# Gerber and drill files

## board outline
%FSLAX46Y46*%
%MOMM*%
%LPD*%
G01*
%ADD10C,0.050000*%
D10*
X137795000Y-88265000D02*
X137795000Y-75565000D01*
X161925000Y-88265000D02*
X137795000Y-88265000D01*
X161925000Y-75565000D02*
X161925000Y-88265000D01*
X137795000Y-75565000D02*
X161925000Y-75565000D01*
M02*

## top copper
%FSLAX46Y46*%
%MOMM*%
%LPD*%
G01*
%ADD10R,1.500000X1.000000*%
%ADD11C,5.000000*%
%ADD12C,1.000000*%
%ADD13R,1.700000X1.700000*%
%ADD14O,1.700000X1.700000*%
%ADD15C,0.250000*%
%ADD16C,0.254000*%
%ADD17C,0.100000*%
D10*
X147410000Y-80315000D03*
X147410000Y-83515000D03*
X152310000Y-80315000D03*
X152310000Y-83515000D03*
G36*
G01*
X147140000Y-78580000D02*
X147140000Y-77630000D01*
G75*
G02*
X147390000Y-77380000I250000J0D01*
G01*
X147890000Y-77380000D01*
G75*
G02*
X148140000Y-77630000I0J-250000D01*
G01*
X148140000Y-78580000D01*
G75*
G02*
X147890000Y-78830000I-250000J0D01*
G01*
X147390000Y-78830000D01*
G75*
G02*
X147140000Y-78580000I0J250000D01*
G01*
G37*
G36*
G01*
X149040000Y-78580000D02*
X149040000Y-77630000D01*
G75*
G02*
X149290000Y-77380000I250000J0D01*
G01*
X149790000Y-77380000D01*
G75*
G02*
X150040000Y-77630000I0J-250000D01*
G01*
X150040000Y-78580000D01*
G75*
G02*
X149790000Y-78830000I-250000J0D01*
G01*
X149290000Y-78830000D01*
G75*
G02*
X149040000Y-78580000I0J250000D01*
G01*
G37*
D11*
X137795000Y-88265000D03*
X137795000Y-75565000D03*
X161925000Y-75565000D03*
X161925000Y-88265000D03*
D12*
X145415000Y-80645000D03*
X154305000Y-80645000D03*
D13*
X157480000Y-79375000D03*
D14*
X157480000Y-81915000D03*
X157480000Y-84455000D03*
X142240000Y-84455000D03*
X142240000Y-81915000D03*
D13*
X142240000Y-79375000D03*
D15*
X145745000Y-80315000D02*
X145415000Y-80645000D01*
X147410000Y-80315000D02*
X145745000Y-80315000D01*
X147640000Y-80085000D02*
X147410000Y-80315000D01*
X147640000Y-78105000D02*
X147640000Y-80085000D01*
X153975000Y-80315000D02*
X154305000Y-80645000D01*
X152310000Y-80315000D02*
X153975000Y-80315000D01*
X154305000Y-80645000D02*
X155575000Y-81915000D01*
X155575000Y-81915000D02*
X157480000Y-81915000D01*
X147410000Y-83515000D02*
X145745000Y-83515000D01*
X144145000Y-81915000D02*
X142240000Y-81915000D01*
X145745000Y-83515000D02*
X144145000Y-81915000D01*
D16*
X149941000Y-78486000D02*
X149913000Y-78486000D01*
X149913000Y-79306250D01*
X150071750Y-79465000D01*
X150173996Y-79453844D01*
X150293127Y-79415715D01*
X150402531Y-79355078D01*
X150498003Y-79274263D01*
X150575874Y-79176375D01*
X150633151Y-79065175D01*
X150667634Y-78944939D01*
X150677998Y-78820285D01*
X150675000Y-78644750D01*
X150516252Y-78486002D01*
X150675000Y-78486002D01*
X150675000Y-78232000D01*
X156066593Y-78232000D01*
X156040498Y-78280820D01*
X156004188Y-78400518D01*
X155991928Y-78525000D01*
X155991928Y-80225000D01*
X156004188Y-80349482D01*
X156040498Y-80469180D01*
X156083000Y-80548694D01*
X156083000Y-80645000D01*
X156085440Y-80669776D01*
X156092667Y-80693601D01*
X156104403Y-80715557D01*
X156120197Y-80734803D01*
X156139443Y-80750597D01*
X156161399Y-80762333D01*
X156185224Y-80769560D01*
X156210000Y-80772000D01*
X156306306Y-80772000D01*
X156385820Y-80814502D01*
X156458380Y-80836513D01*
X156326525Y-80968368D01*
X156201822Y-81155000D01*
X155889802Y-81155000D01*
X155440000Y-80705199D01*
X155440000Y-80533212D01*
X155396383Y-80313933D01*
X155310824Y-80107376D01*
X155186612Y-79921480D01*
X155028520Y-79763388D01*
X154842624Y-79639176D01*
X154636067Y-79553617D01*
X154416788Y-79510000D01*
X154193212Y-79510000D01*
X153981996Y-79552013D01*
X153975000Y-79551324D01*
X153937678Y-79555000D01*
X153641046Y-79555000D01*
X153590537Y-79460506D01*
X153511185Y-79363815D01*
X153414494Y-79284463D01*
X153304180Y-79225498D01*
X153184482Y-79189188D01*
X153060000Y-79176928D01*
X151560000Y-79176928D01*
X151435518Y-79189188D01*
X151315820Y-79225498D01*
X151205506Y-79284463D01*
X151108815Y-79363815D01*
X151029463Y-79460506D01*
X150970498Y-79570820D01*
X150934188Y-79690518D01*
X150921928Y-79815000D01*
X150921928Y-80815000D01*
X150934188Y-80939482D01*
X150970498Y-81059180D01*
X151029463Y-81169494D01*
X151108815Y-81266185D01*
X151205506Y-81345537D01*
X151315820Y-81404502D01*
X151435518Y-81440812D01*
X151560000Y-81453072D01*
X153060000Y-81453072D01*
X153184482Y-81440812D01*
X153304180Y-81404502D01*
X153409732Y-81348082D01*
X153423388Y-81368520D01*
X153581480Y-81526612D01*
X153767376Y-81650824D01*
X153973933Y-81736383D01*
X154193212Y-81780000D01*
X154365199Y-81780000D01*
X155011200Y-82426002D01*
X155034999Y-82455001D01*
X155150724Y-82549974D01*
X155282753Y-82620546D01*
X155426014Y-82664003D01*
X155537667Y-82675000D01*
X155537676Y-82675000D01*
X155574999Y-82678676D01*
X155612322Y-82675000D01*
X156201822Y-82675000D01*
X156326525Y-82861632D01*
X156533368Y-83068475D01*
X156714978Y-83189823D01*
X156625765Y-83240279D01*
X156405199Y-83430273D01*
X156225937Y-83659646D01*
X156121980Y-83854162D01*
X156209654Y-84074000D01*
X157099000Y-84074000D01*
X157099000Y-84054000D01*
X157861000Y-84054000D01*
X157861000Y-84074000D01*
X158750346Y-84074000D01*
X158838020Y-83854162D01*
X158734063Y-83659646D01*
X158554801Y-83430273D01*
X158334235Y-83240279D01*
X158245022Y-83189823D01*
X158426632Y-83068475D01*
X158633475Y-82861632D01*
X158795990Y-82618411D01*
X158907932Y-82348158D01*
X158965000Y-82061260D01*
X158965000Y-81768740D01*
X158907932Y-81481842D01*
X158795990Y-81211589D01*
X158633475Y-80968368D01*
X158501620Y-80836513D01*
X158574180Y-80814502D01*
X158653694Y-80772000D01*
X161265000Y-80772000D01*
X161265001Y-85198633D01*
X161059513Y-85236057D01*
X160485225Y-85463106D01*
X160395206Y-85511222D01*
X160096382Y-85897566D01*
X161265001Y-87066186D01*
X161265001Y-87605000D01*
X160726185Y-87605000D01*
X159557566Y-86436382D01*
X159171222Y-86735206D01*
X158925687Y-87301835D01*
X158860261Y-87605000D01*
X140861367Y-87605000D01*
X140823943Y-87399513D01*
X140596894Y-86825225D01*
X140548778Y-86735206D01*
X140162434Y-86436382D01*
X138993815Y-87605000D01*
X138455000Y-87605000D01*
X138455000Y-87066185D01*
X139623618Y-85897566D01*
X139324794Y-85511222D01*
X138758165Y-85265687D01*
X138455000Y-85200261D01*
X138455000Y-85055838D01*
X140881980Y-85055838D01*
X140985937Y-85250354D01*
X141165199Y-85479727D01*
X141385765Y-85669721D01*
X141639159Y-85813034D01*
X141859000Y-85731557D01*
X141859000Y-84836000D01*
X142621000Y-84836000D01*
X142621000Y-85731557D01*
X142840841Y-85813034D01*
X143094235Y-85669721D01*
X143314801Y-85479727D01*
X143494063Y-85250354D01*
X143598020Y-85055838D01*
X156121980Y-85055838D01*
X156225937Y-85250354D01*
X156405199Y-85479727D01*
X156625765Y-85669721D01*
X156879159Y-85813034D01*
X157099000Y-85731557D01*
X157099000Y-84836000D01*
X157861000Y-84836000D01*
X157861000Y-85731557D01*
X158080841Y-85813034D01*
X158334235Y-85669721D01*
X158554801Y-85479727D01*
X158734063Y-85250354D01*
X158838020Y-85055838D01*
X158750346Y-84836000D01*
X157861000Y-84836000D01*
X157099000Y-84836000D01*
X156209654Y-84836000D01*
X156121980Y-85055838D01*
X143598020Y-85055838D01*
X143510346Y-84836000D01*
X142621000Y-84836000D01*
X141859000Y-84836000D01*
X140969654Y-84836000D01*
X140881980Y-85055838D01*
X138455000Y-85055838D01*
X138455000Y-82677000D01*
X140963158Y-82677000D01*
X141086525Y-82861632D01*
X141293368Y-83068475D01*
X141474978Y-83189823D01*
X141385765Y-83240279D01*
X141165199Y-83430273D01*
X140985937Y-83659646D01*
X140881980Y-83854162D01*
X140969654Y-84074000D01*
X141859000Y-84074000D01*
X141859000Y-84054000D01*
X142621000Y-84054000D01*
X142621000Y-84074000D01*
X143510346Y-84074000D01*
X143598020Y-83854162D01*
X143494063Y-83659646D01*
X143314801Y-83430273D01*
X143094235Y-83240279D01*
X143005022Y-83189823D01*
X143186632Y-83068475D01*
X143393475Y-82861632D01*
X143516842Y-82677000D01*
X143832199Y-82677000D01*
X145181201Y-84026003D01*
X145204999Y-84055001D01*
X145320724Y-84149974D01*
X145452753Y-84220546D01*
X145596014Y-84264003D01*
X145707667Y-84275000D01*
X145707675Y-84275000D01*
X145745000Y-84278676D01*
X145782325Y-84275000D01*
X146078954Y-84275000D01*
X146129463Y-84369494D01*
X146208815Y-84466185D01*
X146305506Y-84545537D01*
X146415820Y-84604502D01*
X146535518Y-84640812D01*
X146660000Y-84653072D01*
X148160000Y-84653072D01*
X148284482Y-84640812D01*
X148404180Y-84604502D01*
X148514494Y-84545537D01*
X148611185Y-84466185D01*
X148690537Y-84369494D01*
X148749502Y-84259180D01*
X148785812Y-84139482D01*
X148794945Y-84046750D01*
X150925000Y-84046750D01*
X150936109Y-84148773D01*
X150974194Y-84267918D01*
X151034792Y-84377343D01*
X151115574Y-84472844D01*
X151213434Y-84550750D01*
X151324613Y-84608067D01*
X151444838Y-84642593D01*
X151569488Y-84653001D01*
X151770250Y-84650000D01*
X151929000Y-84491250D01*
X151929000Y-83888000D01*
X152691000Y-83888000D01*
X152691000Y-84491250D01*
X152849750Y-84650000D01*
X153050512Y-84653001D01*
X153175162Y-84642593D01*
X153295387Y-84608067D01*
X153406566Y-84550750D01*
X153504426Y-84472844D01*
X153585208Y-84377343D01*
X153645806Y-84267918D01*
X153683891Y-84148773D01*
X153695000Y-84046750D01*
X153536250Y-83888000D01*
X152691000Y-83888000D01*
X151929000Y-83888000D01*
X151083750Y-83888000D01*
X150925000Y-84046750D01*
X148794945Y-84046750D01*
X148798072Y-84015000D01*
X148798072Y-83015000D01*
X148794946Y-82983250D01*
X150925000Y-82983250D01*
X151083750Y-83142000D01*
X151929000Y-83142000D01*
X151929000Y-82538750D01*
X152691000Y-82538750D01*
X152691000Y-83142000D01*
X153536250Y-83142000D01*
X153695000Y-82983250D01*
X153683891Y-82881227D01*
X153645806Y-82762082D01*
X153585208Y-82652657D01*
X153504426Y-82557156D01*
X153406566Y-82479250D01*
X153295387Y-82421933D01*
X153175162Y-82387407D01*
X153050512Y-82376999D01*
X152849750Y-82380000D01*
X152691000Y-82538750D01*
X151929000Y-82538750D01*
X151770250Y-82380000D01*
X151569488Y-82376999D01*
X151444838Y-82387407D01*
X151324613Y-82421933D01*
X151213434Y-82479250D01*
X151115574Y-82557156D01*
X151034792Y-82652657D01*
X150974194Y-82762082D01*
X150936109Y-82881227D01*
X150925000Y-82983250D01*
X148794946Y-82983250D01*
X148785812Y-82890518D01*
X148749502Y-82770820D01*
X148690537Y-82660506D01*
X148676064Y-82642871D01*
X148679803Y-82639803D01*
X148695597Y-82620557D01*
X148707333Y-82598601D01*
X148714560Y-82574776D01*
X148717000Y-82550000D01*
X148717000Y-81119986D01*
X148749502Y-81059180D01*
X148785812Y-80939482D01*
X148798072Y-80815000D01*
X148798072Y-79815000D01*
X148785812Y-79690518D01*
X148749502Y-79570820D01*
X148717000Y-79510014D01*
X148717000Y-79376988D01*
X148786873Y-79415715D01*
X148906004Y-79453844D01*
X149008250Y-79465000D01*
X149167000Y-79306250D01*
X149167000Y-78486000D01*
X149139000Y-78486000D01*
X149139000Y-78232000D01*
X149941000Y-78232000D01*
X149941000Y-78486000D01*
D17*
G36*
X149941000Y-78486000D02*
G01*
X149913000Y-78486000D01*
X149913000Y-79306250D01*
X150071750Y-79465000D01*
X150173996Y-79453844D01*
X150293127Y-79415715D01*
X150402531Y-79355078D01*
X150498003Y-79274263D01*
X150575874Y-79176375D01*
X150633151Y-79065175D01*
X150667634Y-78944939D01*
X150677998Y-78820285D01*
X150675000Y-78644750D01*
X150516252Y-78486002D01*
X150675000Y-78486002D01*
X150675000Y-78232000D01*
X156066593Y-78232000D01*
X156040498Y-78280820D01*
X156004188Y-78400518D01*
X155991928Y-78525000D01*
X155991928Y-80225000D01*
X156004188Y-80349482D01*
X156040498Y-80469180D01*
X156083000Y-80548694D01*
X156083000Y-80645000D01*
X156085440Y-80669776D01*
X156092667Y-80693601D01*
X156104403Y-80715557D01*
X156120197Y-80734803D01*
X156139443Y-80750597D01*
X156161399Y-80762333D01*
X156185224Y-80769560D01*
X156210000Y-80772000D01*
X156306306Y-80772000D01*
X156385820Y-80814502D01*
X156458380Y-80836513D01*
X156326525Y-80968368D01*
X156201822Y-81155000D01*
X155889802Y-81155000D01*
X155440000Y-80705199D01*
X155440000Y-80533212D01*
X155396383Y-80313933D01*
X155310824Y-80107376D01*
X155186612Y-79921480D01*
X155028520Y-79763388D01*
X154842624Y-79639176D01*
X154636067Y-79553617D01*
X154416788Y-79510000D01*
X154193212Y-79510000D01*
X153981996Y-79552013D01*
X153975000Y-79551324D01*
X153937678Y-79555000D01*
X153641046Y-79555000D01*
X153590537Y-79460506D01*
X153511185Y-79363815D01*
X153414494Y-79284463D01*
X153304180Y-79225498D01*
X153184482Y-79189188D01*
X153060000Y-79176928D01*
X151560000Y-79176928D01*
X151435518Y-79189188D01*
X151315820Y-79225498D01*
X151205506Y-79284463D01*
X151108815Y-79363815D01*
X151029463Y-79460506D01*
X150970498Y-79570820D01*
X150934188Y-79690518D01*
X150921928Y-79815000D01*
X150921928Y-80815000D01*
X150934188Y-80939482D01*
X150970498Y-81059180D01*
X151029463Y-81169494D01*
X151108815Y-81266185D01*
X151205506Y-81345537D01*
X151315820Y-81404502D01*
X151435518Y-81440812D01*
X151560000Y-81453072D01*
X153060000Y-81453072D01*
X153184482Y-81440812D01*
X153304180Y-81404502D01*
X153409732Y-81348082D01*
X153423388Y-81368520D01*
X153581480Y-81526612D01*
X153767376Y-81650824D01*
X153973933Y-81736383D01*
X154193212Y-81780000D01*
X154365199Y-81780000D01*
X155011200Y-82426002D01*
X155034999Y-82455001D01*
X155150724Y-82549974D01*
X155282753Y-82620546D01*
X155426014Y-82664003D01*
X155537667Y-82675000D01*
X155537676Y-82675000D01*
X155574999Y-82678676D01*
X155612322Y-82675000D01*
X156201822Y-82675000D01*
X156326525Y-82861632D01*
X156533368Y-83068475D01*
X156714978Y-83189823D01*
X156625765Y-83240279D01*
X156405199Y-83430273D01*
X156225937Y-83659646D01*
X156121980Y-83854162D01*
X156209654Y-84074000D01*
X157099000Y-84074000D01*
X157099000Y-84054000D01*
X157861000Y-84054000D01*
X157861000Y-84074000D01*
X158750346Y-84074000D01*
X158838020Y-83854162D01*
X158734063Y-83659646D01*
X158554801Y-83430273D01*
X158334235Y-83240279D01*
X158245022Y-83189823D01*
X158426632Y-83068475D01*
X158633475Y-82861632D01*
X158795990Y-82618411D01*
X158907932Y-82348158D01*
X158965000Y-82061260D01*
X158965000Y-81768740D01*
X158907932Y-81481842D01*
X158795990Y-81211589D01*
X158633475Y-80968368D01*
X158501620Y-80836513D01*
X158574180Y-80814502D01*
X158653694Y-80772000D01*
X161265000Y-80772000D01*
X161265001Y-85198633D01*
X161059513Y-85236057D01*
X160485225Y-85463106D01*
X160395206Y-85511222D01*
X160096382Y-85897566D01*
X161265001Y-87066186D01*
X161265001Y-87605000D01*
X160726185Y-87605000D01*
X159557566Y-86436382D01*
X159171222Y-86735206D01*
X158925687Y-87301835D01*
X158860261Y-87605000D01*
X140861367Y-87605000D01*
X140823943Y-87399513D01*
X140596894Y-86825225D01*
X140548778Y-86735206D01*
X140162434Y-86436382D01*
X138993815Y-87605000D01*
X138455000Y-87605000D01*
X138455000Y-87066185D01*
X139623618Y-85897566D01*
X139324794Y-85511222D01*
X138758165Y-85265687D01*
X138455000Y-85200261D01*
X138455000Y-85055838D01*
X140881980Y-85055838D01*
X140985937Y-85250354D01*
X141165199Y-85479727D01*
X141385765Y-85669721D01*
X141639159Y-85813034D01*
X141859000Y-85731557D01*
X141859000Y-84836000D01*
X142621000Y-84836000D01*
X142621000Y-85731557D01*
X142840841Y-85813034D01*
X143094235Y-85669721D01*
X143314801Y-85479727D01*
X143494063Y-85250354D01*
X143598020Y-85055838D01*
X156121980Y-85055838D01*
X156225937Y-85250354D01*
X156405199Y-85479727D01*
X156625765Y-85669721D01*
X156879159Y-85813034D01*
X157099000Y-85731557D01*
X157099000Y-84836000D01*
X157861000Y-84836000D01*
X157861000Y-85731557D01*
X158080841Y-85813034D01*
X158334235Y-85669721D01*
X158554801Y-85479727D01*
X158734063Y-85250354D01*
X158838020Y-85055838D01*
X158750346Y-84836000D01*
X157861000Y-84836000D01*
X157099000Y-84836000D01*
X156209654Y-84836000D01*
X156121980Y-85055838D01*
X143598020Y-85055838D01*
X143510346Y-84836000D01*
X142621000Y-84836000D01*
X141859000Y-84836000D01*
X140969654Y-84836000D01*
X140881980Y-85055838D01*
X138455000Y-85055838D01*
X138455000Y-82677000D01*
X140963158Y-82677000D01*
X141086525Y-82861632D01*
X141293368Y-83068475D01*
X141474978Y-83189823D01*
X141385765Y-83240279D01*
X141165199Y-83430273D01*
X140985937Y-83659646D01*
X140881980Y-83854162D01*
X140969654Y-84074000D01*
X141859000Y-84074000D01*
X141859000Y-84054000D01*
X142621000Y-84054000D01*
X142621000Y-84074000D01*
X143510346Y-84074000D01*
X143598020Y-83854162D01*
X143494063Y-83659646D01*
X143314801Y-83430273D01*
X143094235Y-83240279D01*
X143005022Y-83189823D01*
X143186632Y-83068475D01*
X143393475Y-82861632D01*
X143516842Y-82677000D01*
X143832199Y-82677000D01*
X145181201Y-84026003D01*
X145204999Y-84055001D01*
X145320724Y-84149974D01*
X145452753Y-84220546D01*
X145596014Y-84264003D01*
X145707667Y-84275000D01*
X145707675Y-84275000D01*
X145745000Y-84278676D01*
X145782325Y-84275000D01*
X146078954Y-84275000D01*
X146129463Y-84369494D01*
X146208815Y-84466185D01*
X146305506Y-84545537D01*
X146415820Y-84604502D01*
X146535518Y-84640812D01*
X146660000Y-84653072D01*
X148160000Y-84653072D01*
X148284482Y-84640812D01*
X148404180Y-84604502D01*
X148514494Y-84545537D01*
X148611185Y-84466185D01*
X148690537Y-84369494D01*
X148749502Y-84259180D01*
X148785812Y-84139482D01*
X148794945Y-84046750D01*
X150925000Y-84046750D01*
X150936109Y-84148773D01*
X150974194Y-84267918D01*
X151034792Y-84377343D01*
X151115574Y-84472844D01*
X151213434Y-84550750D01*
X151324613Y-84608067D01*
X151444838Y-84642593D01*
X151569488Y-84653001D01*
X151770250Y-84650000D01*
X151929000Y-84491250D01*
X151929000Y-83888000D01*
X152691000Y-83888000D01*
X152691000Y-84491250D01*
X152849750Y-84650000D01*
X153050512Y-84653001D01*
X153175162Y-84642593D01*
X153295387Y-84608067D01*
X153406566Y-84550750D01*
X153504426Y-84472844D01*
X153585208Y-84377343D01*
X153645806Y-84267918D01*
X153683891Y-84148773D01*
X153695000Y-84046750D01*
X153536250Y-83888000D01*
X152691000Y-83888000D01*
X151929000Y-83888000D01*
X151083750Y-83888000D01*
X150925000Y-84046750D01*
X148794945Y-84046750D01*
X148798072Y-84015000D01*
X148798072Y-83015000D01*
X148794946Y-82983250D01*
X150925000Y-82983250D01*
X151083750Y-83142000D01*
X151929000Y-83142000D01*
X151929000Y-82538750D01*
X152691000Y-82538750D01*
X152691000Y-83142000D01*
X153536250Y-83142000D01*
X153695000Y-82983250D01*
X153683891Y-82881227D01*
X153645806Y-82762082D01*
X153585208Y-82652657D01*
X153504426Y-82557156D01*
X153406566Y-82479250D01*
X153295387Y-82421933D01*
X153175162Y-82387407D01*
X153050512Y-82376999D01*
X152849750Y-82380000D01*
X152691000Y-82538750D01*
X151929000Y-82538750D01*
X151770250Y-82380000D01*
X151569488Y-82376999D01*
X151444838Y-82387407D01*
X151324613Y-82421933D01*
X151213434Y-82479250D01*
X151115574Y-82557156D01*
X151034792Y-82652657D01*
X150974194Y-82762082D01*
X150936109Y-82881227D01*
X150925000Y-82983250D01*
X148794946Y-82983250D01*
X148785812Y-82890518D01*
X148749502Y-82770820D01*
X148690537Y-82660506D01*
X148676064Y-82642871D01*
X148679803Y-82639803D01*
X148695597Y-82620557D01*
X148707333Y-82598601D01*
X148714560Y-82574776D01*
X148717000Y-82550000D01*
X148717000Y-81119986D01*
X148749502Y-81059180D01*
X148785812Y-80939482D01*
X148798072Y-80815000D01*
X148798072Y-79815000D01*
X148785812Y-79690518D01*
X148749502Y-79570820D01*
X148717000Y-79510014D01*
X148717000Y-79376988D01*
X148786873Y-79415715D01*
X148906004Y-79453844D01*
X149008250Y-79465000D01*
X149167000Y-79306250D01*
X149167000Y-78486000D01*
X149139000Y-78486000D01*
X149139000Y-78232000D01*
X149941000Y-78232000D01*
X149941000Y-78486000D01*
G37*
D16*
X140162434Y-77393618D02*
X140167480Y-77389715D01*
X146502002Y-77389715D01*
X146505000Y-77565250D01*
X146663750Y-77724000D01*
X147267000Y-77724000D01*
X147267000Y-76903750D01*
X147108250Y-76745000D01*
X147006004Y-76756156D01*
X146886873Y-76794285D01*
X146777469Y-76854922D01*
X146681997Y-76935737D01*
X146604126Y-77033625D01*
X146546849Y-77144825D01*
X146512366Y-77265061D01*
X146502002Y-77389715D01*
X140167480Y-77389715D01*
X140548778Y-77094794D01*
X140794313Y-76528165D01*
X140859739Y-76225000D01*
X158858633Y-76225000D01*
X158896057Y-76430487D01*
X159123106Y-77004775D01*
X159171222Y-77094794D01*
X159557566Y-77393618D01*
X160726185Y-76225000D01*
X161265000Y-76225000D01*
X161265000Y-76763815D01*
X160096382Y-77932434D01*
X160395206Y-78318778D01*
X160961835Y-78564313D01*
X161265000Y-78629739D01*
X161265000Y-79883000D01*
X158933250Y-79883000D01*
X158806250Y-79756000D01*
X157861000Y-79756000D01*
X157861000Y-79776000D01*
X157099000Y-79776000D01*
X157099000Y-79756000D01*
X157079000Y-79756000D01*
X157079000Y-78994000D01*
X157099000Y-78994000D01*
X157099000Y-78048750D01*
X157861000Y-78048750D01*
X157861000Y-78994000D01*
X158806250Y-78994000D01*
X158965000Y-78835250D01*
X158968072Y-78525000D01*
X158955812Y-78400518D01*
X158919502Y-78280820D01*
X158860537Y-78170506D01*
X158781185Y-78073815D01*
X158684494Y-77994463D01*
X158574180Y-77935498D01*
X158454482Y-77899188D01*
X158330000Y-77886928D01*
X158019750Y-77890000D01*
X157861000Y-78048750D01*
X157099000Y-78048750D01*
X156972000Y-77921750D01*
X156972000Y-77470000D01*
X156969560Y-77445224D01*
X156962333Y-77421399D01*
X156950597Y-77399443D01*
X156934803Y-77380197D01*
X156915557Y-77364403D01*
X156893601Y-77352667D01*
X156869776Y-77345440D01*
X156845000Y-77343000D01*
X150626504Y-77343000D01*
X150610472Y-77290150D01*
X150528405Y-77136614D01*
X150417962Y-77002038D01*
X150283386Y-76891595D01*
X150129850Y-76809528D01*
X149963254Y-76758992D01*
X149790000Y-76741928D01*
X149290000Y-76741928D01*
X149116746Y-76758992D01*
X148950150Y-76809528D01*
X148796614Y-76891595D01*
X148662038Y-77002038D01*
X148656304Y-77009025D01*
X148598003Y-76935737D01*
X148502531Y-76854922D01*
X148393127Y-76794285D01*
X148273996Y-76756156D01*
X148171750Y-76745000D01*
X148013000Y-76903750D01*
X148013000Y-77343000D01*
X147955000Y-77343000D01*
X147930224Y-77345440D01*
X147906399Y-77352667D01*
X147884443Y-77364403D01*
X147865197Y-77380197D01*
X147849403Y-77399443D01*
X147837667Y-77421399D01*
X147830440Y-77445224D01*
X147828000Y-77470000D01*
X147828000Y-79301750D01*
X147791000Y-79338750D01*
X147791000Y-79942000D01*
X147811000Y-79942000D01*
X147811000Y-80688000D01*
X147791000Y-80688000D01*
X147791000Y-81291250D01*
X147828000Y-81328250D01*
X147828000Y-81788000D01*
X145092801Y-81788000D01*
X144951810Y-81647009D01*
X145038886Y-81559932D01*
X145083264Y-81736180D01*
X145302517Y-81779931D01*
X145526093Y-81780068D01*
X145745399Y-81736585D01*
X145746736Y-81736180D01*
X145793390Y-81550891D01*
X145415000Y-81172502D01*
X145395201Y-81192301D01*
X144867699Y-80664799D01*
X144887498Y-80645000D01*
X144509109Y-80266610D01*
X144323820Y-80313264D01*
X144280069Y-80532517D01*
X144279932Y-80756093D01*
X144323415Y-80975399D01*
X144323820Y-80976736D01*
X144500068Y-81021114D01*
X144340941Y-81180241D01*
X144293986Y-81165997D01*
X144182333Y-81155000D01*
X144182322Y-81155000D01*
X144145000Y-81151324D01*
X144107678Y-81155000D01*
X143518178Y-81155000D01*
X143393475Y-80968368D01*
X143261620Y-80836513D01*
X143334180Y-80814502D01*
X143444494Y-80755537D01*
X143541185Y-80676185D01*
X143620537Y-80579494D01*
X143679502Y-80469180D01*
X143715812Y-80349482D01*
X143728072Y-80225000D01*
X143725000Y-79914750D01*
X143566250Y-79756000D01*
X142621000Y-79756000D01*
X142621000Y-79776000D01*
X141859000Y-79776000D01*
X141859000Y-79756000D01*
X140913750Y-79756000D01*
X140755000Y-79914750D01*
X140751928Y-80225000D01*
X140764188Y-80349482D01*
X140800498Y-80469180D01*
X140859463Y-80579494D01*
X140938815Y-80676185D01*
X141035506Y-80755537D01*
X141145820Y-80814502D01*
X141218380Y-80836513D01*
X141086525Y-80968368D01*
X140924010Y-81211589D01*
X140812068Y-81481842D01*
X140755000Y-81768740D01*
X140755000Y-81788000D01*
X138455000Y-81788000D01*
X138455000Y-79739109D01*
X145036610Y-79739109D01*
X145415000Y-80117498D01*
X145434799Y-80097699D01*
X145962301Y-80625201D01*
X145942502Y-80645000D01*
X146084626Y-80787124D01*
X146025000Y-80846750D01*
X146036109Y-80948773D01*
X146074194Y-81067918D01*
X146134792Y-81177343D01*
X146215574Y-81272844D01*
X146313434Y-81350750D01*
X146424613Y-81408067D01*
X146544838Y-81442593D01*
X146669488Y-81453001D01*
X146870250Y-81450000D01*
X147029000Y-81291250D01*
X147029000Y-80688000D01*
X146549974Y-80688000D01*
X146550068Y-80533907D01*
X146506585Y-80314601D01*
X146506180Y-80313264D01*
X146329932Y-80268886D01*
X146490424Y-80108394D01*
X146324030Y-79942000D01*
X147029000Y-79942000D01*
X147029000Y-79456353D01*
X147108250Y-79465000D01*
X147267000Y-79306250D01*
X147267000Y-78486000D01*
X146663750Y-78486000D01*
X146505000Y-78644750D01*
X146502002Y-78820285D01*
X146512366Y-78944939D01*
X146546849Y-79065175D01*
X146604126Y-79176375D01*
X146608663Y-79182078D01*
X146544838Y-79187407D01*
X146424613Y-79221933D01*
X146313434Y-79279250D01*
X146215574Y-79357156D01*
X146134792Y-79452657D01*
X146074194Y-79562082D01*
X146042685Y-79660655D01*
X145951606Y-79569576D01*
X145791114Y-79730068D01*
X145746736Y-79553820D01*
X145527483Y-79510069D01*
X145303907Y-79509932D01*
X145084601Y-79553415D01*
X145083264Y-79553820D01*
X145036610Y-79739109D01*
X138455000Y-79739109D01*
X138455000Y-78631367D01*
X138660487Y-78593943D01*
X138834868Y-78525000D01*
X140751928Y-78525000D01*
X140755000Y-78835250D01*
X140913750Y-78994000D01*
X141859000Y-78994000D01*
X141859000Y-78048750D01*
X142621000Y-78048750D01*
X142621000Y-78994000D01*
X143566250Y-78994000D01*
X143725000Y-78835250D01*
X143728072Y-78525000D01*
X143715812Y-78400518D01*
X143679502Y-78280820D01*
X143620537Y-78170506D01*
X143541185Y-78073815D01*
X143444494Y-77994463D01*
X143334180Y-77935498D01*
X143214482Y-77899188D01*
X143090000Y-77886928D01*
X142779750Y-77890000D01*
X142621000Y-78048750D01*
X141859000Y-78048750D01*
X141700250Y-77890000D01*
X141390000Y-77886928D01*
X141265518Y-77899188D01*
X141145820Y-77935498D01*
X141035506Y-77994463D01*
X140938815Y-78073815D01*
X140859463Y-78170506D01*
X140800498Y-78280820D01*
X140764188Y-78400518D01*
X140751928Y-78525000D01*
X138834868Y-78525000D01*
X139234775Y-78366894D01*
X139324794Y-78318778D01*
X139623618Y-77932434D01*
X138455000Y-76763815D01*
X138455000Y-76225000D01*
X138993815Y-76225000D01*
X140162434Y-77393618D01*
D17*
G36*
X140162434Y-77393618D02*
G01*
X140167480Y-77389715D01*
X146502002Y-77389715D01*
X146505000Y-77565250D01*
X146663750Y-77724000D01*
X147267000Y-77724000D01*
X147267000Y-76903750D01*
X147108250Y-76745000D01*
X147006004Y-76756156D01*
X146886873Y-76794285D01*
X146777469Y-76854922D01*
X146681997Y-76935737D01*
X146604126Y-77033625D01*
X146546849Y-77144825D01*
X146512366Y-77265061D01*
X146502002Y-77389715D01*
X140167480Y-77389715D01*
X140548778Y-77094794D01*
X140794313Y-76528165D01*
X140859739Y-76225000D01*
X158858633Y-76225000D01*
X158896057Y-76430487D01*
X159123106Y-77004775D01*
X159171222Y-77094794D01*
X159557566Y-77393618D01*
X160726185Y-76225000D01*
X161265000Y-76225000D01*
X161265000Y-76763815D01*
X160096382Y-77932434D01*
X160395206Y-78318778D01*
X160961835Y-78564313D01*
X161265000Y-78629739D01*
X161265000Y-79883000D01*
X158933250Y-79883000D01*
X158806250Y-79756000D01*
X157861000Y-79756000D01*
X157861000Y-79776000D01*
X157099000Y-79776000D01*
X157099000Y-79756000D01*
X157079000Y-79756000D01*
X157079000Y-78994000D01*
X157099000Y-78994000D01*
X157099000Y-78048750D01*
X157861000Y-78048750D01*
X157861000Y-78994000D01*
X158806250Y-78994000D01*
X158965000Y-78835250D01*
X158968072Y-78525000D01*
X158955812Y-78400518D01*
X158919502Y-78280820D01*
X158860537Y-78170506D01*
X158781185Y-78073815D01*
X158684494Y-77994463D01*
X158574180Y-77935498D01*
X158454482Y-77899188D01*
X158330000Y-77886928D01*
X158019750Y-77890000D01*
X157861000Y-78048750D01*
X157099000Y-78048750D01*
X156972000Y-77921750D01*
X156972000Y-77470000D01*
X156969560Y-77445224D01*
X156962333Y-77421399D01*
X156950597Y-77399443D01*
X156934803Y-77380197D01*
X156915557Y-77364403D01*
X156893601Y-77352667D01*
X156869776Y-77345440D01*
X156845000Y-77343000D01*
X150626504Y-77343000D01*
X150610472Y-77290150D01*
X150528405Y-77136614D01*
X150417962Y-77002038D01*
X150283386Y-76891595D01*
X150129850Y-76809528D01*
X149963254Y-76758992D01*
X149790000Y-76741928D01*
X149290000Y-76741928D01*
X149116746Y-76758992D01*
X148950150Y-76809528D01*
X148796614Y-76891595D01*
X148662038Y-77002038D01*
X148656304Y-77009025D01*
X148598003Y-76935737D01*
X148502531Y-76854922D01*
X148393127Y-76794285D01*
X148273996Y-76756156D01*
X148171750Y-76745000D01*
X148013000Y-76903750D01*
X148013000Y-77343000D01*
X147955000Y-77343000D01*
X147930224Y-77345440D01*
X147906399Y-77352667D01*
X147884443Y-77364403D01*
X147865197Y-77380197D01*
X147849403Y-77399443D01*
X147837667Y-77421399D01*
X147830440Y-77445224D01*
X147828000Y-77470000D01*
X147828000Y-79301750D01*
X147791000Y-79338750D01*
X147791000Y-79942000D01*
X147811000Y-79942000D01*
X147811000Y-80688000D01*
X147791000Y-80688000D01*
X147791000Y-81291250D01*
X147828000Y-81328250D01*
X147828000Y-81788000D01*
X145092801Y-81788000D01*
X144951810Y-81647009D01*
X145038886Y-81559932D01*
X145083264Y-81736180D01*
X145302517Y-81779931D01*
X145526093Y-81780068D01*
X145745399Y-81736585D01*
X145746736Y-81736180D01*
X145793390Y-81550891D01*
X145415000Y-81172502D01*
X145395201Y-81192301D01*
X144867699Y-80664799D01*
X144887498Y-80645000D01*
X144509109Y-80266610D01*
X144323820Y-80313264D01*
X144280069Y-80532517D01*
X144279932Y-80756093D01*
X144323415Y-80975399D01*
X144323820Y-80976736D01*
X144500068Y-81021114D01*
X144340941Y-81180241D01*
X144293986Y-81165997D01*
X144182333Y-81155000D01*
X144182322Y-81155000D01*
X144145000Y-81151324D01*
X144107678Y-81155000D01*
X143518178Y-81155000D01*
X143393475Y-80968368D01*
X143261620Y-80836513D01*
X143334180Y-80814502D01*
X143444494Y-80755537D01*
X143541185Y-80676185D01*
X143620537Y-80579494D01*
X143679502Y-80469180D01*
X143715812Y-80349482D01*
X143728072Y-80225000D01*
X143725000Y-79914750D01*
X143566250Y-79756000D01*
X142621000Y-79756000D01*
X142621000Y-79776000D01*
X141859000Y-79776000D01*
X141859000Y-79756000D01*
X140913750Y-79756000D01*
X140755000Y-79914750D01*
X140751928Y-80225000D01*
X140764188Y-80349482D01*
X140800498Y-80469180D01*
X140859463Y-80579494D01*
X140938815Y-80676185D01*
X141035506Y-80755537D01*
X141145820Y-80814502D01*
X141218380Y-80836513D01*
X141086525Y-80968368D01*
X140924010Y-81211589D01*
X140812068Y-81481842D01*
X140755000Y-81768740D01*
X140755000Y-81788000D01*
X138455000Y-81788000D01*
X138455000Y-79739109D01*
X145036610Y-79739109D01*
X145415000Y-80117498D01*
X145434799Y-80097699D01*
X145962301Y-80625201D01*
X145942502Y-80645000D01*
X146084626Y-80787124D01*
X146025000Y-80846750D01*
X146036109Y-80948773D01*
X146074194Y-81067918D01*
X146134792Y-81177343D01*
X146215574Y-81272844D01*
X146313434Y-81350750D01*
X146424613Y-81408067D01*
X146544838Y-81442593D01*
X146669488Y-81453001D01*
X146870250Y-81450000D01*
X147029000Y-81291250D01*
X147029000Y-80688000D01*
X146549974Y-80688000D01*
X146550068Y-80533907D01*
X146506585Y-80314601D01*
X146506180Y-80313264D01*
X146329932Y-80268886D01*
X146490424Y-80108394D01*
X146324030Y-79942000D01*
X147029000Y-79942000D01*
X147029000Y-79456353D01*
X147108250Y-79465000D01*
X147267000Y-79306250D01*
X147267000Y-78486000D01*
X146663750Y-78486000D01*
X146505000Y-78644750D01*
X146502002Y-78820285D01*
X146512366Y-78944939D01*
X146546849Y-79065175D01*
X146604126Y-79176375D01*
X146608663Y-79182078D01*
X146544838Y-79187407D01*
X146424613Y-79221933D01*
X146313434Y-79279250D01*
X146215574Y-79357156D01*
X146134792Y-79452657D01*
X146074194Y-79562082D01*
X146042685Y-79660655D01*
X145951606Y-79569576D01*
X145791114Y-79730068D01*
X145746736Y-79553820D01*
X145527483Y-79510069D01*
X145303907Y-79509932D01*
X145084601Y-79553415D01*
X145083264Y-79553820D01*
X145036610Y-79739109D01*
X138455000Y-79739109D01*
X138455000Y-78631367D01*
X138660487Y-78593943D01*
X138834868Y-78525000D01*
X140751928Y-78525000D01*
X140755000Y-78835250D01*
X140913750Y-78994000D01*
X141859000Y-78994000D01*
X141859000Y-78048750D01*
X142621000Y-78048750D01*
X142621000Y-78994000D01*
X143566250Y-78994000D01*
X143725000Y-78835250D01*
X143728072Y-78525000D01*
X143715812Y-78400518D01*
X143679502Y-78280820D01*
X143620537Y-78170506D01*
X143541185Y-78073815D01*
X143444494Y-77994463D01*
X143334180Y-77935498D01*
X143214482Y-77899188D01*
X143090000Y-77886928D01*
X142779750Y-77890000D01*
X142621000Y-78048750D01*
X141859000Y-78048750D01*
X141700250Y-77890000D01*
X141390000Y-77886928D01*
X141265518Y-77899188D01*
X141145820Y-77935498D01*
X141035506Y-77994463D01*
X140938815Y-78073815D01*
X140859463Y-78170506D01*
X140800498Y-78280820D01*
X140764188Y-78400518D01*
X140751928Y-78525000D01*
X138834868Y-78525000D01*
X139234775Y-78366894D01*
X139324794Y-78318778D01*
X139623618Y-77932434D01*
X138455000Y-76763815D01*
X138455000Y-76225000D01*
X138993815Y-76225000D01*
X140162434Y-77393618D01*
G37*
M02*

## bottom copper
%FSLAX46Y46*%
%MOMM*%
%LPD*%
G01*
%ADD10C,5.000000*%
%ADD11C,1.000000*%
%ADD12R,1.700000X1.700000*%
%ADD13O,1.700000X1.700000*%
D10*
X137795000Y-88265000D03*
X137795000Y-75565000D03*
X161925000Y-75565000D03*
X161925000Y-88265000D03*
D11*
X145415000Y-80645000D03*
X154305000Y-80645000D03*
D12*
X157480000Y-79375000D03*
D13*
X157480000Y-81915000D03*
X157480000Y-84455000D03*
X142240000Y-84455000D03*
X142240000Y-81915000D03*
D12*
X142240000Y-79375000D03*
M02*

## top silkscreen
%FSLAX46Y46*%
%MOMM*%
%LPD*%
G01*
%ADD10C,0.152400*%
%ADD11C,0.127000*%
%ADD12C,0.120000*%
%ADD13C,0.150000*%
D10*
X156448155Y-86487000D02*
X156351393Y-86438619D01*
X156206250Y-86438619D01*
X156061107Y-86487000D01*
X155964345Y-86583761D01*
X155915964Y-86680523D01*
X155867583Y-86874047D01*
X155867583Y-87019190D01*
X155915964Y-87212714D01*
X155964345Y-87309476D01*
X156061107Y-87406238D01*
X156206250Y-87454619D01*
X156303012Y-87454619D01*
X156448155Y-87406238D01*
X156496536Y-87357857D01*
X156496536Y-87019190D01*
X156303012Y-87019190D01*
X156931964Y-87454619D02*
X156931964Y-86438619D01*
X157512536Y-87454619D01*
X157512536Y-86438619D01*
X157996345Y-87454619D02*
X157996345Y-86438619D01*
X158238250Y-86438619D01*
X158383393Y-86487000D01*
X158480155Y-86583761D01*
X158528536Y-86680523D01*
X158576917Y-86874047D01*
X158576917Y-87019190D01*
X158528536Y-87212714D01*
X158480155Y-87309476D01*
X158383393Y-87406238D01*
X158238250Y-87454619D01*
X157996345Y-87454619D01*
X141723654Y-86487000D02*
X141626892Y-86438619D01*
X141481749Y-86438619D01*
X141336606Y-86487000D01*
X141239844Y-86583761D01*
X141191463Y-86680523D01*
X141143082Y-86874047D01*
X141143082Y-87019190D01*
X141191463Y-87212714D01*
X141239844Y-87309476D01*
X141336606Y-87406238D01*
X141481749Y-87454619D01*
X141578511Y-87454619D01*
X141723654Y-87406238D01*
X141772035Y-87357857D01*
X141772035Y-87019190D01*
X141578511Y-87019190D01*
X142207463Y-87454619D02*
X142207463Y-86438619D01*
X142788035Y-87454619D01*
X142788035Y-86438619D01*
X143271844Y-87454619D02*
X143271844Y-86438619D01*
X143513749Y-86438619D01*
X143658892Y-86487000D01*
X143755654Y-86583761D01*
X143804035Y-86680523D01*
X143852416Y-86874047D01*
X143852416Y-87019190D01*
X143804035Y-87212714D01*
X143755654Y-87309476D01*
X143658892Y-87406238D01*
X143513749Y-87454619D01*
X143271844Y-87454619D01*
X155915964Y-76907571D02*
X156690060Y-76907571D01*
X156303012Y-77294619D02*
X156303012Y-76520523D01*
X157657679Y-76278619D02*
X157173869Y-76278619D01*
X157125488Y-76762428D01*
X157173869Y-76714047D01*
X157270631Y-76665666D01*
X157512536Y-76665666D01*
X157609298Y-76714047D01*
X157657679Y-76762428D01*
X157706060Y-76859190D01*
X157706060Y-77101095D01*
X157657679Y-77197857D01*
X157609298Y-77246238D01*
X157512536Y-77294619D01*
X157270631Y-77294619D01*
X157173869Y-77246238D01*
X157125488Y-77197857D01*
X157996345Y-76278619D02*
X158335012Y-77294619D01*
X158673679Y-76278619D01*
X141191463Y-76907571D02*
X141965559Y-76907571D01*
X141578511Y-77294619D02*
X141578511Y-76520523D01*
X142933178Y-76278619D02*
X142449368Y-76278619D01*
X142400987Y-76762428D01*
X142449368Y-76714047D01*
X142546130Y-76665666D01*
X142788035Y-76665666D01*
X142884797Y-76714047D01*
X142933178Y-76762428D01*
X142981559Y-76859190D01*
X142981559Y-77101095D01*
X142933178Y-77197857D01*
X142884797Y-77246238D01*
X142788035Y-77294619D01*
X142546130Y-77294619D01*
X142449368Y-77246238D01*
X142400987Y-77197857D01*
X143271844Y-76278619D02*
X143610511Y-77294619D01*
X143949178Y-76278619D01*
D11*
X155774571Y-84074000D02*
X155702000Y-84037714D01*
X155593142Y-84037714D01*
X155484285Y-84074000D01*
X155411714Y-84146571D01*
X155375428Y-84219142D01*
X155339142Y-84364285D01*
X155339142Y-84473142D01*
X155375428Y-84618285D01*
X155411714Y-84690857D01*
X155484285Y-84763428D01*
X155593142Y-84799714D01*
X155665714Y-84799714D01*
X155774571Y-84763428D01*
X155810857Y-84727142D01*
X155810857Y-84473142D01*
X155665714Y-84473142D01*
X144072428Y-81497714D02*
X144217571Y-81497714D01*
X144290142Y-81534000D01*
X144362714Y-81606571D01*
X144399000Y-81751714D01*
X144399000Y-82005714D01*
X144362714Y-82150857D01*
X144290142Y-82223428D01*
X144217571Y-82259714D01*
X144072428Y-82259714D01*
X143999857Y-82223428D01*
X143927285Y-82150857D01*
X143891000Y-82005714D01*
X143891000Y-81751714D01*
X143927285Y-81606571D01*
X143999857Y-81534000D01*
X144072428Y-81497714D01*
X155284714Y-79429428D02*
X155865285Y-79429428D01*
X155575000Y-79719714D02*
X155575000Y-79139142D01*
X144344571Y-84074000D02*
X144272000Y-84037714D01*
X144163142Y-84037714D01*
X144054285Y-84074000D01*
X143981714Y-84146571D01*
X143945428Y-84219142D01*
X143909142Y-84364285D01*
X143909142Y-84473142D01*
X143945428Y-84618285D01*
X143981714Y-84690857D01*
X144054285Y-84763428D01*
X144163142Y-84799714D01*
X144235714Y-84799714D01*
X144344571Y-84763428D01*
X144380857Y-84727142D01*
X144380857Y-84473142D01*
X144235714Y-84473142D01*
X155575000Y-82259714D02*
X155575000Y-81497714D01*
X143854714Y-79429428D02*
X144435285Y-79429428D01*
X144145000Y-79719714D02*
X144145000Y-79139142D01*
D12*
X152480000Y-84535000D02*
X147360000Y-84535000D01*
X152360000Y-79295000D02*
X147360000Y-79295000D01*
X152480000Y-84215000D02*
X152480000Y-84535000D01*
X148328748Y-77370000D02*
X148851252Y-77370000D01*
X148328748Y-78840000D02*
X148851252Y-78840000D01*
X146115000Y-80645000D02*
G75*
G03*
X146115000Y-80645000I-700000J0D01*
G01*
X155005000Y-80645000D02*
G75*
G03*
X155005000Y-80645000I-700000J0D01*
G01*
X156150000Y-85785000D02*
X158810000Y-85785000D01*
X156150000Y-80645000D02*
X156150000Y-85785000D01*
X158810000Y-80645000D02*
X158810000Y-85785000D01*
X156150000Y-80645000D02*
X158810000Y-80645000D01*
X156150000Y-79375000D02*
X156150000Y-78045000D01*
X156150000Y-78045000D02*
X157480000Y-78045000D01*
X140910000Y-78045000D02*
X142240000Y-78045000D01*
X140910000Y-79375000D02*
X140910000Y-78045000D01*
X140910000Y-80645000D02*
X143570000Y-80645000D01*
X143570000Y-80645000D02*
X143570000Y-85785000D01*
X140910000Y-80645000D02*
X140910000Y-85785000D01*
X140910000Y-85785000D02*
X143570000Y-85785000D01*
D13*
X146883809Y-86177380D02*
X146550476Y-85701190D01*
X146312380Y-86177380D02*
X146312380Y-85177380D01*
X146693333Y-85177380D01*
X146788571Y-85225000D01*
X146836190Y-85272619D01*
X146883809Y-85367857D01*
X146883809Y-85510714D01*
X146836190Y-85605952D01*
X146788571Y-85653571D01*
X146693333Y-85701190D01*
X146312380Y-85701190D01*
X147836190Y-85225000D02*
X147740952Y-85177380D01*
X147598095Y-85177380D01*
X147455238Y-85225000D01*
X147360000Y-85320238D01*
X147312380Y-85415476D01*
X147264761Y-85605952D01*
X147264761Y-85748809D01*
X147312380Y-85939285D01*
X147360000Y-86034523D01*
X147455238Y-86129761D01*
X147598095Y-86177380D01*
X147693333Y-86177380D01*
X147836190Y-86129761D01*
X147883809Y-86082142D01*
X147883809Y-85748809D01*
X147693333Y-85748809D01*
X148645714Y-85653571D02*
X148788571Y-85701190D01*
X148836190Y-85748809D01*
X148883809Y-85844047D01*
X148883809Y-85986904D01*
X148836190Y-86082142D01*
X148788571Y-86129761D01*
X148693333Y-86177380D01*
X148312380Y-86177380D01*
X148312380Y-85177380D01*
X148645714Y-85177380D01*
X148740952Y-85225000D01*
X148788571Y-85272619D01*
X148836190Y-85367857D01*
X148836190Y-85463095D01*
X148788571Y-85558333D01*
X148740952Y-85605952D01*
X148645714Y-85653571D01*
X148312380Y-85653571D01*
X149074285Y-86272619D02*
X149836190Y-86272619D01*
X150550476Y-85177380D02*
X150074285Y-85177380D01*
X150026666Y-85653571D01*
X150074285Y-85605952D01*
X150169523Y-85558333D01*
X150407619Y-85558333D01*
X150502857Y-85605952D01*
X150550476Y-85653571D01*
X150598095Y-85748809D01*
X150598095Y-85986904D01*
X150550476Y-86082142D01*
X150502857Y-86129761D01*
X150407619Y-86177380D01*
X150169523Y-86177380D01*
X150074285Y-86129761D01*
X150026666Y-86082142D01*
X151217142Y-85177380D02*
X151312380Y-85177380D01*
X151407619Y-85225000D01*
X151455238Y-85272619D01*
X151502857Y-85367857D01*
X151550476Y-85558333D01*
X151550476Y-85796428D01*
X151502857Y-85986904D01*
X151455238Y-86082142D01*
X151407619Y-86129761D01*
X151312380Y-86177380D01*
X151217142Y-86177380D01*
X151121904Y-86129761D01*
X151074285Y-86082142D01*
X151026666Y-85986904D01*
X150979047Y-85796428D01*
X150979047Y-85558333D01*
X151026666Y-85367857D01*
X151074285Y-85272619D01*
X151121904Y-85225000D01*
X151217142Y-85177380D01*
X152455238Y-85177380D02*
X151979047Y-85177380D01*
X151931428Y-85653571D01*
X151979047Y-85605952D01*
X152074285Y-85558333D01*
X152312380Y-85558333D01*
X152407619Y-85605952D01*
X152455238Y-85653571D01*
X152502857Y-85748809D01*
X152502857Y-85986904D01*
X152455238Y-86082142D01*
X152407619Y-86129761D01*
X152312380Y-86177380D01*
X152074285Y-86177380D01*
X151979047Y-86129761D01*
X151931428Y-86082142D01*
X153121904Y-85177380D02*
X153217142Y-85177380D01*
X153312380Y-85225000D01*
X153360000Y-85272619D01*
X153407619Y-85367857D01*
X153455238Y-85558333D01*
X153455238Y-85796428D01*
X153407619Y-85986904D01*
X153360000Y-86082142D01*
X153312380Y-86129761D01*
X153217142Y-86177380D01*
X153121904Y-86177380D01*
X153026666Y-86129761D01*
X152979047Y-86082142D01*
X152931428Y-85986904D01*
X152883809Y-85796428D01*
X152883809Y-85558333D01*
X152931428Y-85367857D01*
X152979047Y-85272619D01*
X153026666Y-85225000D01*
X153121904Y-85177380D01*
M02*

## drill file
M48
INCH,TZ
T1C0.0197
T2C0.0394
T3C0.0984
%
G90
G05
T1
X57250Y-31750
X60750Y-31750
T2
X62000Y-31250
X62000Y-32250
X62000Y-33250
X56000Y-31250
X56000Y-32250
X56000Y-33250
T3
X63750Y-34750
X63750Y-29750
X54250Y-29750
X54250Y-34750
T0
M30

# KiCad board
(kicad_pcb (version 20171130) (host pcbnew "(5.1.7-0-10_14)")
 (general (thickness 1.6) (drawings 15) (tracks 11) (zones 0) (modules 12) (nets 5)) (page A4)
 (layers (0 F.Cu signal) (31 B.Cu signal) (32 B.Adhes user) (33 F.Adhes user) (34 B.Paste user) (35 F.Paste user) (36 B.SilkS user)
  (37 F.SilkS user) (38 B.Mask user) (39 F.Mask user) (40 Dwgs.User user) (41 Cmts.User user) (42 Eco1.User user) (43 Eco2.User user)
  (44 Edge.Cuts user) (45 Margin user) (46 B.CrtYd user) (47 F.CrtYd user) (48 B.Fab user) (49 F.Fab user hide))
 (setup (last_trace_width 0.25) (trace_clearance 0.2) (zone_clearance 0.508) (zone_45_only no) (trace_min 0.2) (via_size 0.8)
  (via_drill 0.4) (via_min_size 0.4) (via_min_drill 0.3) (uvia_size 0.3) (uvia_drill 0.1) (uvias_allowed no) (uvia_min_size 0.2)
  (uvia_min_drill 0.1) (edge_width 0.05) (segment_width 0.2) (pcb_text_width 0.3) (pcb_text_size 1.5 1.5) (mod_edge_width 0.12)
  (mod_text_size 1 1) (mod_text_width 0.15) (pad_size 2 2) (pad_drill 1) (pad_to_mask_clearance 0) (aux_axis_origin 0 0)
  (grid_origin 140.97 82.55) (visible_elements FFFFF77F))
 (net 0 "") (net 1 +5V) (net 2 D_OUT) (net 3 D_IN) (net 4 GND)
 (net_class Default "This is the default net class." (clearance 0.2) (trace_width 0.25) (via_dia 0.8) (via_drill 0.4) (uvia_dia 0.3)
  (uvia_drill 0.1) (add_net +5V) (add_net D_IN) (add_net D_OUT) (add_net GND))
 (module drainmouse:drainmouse (layer F.Cu) (at 144.78 85.725)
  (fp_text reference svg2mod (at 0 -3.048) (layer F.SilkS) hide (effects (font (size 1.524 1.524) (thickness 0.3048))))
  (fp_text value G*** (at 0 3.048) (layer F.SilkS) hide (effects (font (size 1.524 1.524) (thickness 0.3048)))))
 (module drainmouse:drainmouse (layer F.Cu) (at 139.065 83.82)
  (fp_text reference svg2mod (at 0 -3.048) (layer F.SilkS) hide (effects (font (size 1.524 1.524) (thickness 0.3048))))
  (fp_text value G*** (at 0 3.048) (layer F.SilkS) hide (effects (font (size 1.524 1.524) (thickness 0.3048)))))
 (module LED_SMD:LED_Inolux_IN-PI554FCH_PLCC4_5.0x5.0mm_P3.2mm (layer F.Cu) (at 149.86 81.915 180)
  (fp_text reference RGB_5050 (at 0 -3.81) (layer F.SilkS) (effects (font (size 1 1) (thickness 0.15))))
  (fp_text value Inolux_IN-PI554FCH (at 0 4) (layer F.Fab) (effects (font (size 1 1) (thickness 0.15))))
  (fp_line (start -2.62 -2.62) (end 2.5 -2.62) (layer F.SilkS) (width 0.12))
  (fp_line (start -2.5 2.62) (end 2.5 2.62) (layer F.SilkS) (width 0.12))
  (fp_line (start -2.62 -2.3) (end -2.62 -2.62) (layer F.SilkS) (width 0.12))
  (pad 3 smd rect (at 2.45 1.6 180) (size 1.5 1) (layers F.Cu F.Paste F.Mask) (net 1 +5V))
  (pad 4 smd rect (at 2.45 -1.6 180) (size 1.5 1) (layers F.Cu F.Paste F.Mask) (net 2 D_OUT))
  (pad 2 smd rect (at -2.45 1.6 180) (size 1.5 1) (layers F.Cu F.Paste F.Mask) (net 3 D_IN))
  (pad 1 smd rect (at -2.45 -1.6 180) (size 1.5 1) (layers F.Cu F.Paste F.Mask) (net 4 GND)))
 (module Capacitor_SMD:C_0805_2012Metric (layer F.Cu) (at 148.59 78.105)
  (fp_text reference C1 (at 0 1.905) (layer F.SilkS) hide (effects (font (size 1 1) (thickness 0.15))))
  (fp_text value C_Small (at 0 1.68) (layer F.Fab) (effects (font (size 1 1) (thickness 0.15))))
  (fp_line (start -0.261252 -0.735) (end 0.261252 -0.735) (layer F.SilkS) (width 0.12))
  (fp_line (start -0.261252 0.735) (end 0.261252 0.735) (layer F.SilkS) (width 0.12))
  (pad 1 smd roundrect (at -0.95 0) (size 1 1.45) (layers F.Cu F.Paste F.Mask) (roundrect_rratio 0.25) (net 1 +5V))
  (pad 2 smd roundrect (at 0.95 0) (size 1 1.45) (layers F.Cu F.Paste F.Mask) (roundrect_rratio 0.25) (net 4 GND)))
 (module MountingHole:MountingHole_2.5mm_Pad (layer F.Cu) (at 137.795 88.265)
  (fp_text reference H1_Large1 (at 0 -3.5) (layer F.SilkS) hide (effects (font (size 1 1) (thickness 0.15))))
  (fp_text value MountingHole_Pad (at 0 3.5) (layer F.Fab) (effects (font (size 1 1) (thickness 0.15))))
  (pad 1 thru_hole circle (at 0 0) (size 5 5) (drill 2.5) (layers *.Cu *.Mask) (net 4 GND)))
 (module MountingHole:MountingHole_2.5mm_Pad (layer F.Cu) (at 137.795 75.565)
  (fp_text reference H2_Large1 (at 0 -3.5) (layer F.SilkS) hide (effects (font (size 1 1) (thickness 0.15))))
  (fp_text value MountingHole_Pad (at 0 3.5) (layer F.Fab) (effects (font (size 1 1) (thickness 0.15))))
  (pad 1 thru_hole circle (at 0 0) (size 5 5) (drill 2.5) (layers *.Cu *.Mask) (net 1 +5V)))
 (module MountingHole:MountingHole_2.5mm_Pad (layer F.Cu) (at 161.925 75.565)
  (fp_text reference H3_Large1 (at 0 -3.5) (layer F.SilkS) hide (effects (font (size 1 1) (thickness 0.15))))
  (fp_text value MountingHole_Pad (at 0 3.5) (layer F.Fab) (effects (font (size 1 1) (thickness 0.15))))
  (pad 1 thru_hole circle (at 0 0) (size 5 5) (drill 2.5) (layers *.Cu *.Mask) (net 1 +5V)))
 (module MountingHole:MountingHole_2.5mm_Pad (layer F.Cu) (at 161.925 88.265)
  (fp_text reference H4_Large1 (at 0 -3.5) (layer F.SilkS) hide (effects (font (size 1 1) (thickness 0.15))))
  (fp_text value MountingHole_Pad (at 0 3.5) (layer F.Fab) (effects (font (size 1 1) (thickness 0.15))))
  (pad 1 thru_hole circle (at 0 0) (size 5 5) (drill 2.5) (layers *.Cu *.Mask) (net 4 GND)))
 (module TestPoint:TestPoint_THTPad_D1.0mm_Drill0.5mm (layer F.Cu) (at 145.415 80.645)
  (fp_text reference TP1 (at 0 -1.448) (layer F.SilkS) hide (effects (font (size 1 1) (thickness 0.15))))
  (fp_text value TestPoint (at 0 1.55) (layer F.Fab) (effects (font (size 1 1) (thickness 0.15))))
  (fp_circle (center 0 0) (end 0 0.7) (layer F.SilkS) (width 0.12))
  (pad 1 thru_hole circle (at 0 0) (size 1 1) (drill 0.5) (layers *.Cu *.Mask) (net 1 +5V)))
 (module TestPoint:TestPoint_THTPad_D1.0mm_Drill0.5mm (layer F.Cu) (at 154.305 80.645)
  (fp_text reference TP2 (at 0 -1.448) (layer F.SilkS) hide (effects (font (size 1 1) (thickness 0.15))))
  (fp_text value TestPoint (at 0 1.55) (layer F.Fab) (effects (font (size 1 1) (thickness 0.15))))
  (fp_circle (center 0 0) (end 0 0.7) (layer F.SilkS) (width 0.12))
  (pad 1 thru_hole circle (at 0 0) (size 1 1) (drill 0.5) (layers *.Cu *.Mask) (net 3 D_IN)))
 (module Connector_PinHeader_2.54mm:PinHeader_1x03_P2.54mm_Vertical (layer F.Cu) (at 157.48 79.375)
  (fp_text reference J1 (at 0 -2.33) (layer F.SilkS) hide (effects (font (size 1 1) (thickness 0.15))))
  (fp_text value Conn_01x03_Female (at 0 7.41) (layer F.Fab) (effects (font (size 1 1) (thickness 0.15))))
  (fp_line (start -1.33 6.41) (end 1.33 6.41) (layer F.SilkS) (width 0.12))
  (fp_line (start -1.33 1.27) (end -1.33 6.41) (layer F.SilkS) (width 0.12))
  (fp_line (start 1.33 1.27) (end 1.33 6.41) (layer F.SilkS) (width 0.12))
  (fp_line (start -1.33 1.27) (end 1.33 1.27) (layer F.SilkS) (width 0.12))
  (fp_line (start -1.33 0) (end -1.33 -1.33) (layer F.SilkS) (width 0.12))
  (fp_line (start -1.33 -1.33) (end 0 -1.33) (layer F.SilkS) (width 0.12))
  (pad 1 thru_hole rect (at 0 0) (size 1.7 1.7) (drill 1) (layers *.Cu *.Mask) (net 1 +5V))
  (pad 2 thru_hole oval (at 0 2.54) (size 1.7 1.7) (drill 1) (layers *.Cu *.Mask) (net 3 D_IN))
  (pad 3 thru_hole oval (at 0 5.08) (size 1.7 1.7) (drill 1) (layers *.Cu *.Mask) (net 4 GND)))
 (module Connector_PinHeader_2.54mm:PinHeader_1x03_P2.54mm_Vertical (layer F.Cu) (at 142.24 79.375)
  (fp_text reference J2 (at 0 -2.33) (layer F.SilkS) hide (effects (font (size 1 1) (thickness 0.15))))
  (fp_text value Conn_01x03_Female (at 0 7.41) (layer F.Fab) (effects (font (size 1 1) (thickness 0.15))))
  (fp_line (start -1.33 -1.33) (end 0 -1.33) (layer F.SilkS) (width 0.12))
  (fp_line (start -1.33 0) (end -1.33 -1.33) (layer F.SilkS) (width 0.12))
  (fp_line (start -1.33 1.27) (end 1.33 1.27) (layer F.SilkS) (width 0.12))
  (fp_line (start 1.33 1.27) (end 1.33 6.41) (layer F.SilkS) (width 0.12))
  (fp_line (start -1.33 1.27) (end -1.33 6.41) (layer F.SilkS) (width 0.12))
  (fp_line (start -1.33 6.41) (end 1.33 6.41) (layer F.SilkS) (width 0.12))
  (pad 3 thru_hole oval (at 0 5.08) (size 1.7 1.7) (drill 1) (layers *.Cu *.Mask) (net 4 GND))
  (pad 2 thru_hole oval (at 0 2.54) (size 1.7 1.7) (drill 1) (layers *.Cu *.Mask) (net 2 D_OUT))
  (pad 1 thru_hole rect (at 0 0) (size 1.7 1.7) (drill 1) (layers *.Cu *.Mask) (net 1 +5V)))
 (gr_line (start 137.795 88.265) (end 137.795 75.565) (layer Edge.Cuts) (width 0.05))
 (gr_line (start 161.925 88.265) (end 137.795 88.265) (layer Edge.Cuts) (width 0.05))
 (gr_line (start 161.925 75.565) (end 161.925 88.265) (layer Edge.Cuts) (width 0.05))
 (gr_line (start 137.795 75.565) (end 161.925 75.565) (layer Edge.Cuts) (width 0.05))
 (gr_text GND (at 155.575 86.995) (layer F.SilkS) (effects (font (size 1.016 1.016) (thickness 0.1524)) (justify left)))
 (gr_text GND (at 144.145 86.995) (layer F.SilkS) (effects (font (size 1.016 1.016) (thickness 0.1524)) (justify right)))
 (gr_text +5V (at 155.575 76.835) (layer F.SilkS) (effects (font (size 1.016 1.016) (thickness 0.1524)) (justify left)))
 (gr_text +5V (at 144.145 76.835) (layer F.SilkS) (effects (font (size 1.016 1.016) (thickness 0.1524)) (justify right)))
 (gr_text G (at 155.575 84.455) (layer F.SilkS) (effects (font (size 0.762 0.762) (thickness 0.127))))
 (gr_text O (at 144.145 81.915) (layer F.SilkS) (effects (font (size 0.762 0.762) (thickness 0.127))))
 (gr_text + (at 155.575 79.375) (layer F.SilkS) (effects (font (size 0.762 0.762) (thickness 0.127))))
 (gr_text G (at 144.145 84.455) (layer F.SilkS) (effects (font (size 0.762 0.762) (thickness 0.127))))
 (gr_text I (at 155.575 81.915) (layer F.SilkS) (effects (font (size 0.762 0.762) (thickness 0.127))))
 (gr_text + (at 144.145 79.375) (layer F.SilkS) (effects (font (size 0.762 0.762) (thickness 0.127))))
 (segment (start 145.745 80.315) (end 145.415 80.645) (width 0.25) (layer F.Cu) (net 1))
 (segment (start 147.41 80.315) (end 145.745 80.315) (width 0.25) (layer F.Cu) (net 1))
 (segment (start 147.64 80.085) (end 147.41 80.315) (width 0.25) (layer F.Cu) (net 1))
 (segment (start 147.64 78.105) (end 147.64 80.085) (width 0.25) (layer F.Cu) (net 1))
 (segment (start 153.975 80.315) (end 154.305 80.645) (width 0.25) (layer F.Cu) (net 3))
 (segment (start 152.31 80.315) (end 153.975 80.315) (width 0.25) (layer F.Cu) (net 3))
 (segment (start 154.305 80.645) (end 155.575 81.915) (width 0.25) (layer F.Cu) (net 3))
 (segment (start 155.575 81.915) (end 157.48 81.915) (width 0.25) (layer F.Cu) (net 3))
 (segment (start 147.41 83.515) (end 145.745 83.515) (width 0.25) (layer F.Cu) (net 2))
 (segment (start 144.145 81.915) (end 142.24 81.915) (width 0.25) (layer F.Cu) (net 2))
 (segment (start 145.745 83.515) (end 144.145 81.915) (width 0.25) (layer F.Cu) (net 2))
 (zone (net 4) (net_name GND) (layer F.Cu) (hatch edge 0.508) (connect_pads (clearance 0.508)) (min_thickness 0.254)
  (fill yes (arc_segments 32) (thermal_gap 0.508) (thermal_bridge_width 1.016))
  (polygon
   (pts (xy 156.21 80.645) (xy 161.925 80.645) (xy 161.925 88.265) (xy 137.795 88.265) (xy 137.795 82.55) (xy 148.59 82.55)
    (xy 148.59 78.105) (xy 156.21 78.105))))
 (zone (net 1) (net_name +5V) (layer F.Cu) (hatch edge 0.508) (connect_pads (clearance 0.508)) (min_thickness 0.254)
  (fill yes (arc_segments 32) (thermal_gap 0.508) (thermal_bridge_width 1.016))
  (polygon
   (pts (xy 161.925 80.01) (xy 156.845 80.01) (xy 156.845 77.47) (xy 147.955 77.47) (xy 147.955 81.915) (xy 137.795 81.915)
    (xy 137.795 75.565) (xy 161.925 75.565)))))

